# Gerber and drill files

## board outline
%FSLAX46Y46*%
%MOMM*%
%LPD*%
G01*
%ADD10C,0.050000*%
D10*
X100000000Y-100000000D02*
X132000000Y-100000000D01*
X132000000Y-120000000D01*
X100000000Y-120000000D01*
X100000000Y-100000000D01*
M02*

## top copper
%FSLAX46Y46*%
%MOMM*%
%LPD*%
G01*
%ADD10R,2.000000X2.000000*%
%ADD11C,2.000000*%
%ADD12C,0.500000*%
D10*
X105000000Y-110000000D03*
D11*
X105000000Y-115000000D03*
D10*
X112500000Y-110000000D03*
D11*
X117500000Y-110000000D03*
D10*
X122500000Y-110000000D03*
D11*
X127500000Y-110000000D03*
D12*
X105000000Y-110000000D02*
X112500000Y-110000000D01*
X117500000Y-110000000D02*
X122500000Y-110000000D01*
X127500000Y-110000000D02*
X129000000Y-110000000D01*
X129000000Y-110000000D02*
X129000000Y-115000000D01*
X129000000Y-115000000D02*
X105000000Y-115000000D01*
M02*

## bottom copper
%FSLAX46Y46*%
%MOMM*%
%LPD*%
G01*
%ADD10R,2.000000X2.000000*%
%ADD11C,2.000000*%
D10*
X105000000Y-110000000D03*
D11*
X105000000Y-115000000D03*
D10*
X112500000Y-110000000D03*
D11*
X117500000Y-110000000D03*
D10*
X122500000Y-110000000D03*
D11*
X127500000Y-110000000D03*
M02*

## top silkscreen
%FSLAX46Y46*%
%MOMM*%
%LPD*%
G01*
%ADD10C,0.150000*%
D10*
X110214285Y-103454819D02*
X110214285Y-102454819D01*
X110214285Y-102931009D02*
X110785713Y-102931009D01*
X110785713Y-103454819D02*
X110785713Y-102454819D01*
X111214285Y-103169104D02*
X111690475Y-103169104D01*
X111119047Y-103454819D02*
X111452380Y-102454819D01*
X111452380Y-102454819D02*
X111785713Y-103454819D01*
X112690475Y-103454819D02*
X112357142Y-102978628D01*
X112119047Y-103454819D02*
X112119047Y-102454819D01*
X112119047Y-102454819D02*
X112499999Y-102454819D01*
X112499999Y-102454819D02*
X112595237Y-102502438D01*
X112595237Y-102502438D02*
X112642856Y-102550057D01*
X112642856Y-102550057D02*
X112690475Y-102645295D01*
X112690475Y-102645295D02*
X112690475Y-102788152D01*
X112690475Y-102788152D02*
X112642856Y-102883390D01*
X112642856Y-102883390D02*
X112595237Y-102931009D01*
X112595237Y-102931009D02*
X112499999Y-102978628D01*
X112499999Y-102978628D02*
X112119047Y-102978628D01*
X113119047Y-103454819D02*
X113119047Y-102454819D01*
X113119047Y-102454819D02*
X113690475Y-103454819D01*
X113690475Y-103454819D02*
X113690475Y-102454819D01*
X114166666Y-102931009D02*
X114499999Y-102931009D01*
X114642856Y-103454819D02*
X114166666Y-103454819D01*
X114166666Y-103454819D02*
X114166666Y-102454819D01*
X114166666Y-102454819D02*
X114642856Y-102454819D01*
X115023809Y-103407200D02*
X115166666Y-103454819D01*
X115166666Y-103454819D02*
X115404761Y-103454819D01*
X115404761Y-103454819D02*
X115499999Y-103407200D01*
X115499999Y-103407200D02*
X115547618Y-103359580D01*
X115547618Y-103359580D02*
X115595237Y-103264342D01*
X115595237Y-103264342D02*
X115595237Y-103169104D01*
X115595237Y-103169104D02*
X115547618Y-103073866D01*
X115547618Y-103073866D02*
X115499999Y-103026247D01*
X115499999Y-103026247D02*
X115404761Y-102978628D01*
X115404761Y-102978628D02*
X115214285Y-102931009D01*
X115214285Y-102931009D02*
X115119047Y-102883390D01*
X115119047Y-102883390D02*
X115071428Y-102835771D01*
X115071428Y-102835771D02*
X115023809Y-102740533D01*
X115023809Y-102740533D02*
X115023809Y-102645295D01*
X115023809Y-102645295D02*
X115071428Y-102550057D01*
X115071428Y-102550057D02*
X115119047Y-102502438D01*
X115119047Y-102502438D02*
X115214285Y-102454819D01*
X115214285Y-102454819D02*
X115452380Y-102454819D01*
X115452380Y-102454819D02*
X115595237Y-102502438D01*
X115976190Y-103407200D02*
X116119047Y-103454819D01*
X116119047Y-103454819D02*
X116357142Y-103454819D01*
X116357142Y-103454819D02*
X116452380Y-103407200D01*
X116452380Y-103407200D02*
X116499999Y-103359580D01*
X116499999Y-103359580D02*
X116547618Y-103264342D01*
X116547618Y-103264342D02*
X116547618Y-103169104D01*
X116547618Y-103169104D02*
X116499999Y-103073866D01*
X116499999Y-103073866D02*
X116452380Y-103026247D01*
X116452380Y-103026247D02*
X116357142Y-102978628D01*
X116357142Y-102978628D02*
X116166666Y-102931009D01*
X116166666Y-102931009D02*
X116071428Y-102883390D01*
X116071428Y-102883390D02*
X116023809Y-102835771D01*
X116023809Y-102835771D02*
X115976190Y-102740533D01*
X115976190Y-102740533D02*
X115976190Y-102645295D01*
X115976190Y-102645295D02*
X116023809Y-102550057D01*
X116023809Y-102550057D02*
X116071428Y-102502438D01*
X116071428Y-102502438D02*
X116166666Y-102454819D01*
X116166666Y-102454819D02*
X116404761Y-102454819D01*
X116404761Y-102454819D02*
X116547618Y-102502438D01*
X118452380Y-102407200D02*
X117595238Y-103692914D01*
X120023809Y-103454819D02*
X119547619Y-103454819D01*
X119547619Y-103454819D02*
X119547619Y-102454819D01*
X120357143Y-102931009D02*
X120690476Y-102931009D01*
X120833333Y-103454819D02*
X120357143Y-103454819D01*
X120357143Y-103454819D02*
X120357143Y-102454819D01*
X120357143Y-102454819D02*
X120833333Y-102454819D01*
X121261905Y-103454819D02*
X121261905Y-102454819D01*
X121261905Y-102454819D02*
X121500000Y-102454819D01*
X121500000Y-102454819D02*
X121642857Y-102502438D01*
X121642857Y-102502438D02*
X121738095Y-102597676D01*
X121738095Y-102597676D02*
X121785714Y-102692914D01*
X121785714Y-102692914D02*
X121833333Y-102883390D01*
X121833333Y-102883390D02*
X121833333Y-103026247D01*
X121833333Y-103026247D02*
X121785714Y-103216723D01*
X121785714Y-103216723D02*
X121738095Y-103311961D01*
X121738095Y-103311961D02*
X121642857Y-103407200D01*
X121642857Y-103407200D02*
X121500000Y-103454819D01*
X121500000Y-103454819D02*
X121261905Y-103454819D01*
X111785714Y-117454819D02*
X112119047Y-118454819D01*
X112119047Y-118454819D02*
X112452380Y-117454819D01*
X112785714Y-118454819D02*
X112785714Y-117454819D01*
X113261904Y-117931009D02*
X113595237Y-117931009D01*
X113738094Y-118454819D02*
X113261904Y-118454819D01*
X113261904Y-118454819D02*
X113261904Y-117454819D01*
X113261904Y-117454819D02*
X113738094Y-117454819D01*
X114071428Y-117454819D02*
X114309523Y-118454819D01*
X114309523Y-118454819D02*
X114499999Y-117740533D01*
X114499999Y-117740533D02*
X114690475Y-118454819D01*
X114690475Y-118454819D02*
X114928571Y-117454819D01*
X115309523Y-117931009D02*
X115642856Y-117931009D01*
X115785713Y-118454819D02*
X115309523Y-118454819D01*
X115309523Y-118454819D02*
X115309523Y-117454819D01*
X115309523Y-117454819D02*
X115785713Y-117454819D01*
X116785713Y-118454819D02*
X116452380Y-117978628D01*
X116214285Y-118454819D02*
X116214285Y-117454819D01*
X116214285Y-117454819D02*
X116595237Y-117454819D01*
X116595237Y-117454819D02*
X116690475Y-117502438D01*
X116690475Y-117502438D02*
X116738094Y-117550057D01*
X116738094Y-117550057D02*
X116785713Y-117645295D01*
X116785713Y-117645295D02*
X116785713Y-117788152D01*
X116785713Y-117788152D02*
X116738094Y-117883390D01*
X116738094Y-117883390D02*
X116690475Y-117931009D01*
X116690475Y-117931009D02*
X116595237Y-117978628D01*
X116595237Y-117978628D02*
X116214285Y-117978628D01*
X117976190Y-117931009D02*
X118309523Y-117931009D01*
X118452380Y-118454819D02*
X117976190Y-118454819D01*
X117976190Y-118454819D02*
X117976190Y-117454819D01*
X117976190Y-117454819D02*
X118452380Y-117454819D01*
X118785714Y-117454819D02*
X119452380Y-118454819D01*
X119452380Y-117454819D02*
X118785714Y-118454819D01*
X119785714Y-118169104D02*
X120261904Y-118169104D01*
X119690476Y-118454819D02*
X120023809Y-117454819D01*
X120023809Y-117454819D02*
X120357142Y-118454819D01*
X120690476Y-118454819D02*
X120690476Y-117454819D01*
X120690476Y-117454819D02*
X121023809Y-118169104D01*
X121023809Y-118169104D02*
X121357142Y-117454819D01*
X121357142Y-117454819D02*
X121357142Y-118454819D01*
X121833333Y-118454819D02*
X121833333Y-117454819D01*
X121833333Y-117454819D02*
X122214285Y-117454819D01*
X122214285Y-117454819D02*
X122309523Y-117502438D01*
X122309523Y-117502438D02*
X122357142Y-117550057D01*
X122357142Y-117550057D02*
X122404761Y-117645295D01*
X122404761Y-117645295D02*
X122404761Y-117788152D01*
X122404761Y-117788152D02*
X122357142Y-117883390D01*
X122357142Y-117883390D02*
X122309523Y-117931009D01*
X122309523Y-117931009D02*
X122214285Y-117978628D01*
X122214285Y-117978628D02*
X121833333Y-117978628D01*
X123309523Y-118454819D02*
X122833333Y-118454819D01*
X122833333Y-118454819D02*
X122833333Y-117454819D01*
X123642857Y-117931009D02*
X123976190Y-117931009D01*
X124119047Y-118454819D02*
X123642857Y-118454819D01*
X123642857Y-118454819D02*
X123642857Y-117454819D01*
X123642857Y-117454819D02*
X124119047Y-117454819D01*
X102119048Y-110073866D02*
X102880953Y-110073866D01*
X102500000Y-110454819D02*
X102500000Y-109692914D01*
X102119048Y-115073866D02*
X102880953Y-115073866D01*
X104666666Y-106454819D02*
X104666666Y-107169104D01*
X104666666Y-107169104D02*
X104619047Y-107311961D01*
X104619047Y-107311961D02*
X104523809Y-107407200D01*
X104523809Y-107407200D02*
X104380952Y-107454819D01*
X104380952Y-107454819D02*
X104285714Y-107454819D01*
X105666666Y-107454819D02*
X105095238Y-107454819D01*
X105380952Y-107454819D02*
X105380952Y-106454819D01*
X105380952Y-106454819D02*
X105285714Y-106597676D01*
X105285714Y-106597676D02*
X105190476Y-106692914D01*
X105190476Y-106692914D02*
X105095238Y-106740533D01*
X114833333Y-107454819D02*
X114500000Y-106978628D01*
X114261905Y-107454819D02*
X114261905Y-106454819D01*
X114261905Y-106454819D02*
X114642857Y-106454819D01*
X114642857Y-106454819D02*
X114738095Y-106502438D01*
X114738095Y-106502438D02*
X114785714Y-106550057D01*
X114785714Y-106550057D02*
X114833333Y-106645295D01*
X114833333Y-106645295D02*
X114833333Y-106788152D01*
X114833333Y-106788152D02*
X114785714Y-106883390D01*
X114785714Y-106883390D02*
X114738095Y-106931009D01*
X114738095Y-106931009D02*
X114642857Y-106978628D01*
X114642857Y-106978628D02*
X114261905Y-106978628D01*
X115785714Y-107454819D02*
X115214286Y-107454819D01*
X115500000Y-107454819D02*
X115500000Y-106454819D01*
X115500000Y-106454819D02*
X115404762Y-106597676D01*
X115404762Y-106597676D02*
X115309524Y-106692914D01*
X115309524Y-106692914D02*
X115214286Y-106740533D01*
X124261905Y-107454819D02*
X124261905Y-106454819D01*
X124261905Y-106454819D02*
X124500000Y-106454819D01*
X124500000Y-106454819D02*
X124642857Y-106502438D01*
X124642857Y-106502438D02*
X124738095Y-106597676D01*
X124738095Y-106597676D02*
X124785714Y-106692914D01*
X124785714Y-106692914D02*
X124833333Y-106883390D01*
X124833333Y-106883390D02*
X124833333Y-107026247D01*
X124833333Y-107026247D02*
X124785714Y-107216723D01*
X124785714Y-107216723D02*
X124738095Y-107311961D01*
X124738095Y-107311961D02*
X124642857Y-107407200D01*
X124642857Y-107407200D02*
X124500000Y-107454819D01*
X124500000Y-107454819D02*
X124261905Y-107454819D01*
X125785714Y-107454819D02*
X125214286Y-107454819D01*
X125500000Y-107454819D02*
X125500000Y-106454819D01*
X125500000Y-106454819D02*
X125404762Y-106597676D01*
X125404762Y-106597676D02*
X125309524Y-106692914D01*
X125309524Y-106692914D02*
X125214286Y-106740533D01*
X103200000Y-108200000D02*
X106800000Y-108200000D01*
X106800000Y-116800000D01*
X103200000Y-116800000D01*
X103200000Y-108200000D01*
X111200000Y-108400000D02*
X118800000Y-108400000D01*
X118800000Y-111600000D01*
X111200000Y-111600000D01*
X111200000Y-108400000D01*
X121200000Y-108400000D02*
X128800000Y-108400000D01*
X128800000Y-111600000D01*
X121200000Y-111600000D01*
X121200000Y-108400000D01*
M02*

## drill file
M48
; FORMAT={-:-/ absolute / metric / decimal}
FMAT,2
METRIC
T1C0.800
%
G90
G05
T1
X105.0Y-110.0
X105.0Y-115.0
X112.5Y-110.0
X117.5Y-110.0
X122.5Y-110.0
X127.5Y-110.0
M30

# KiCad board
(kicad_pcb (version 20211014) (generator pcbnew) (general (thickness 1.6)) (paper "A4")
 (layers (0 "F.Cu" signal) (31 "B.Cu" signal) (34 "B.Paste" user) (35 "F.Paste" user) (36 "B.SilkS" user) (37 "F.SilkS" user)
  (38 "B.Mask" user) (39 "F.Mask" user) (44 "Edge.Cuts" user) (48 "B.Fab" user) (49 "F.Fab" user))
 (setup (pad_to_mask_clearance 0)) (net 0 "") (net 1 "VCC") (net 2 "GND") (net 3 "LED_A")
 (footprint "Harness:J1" (layer "F.Cu") (at 105 110)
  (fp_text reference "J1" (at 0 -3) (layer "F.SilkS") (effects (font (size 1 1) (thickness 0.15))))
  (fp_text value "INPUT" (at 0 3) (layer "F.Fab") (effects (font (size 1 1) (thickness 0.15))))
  (fp_rect (start -1.8 -1.8) (end 1.8 6.8) (layer "F.SilkS") (width 0.15) (fill none))
  (pad "1" thru_hole rect (at 0 0) (size 2 2) (drill 0.8) (layers "*.Cu" "*.Mask") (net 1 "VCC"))
  (pad "2" thru_hole circle (at 0 5) (size 2 2) (drill 0.8) (layers "*.Cu" "*.Mask") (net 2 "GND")))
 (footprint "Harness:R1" (layer "F.Cu") (at 115 110)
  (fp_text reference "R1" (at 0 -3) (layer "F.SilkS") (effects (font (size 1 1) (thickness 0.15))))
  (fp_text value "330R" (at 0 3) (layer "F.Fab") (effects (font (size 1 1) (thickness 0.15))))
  (fp_rect (start -3.8 -1.6) (end 3.8 1.6) (layer "F.SilkS") (width 0.15) (fill none))
  (pad "1" thru_hole rect (at -2.5 0) (size 2 2) (drill 0.8) (layers "*.Cu" "*.Mask") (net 1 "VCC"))
  (pad "2" thru_hole circle (at 2.5 0) (size 2 2) (drill 0.8) (layers "*.Cu" "*.Mask") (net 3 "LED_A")))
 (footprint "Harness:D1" (layer "F.Cu") (at 125 110)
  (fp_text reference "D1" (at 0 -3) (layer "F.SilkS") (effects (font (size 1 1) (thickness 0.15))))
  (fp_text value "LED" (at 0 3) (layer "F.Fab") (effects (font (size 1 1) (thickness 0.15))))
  (fp_rect (start -3.8 -1.6) (end 3.8 1.6) (layer "F.SilkS") (width 0.15) (fill none))
  (pad "1" thru_hole rect (at -2.5 0) (size 2 2) (drill 0.8) (layers "*.Cu" "*.Mask") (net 3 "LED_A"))
  (pad "2" thru_hole circle (at 2.5 0) (size 2 2) (drill 0.8) (layers "*.Cu" "*.Mask") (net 2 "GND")))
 (segment (start 105 110) (end 112.5 110) (width 0.5) (layer "F.Cu") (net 1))
 (segment (start 117.5 110) (end 122.5 110) (width 0.5) (layer "F.Cu") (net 3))
 (segment (start 127.5 110) (end 129 110) (width 0.5) (layer "F.Cu") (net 2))
 (segment (start 129 110) (end 129 115) (width 0.5) (layer "F.Cu") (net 2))
 (segment (start 129 115) (end 105 115) (width 0.5) (layer "F.Cu") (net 2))
 (gr_rect (start 100 100) (end 132 120) (layer "Edge.Cuts") (width 0.05) (fill none))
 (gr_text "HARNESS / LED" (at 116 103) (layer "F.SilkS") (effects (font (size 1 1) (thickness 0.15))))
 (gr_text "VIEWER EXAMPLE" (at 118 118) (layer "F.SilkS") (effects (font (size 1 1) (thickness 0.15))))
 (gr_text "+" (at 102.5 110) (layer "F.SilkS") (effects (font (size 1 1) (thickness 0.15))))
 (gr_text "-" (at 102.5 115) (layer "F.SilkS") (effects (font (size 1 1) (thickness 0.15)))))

